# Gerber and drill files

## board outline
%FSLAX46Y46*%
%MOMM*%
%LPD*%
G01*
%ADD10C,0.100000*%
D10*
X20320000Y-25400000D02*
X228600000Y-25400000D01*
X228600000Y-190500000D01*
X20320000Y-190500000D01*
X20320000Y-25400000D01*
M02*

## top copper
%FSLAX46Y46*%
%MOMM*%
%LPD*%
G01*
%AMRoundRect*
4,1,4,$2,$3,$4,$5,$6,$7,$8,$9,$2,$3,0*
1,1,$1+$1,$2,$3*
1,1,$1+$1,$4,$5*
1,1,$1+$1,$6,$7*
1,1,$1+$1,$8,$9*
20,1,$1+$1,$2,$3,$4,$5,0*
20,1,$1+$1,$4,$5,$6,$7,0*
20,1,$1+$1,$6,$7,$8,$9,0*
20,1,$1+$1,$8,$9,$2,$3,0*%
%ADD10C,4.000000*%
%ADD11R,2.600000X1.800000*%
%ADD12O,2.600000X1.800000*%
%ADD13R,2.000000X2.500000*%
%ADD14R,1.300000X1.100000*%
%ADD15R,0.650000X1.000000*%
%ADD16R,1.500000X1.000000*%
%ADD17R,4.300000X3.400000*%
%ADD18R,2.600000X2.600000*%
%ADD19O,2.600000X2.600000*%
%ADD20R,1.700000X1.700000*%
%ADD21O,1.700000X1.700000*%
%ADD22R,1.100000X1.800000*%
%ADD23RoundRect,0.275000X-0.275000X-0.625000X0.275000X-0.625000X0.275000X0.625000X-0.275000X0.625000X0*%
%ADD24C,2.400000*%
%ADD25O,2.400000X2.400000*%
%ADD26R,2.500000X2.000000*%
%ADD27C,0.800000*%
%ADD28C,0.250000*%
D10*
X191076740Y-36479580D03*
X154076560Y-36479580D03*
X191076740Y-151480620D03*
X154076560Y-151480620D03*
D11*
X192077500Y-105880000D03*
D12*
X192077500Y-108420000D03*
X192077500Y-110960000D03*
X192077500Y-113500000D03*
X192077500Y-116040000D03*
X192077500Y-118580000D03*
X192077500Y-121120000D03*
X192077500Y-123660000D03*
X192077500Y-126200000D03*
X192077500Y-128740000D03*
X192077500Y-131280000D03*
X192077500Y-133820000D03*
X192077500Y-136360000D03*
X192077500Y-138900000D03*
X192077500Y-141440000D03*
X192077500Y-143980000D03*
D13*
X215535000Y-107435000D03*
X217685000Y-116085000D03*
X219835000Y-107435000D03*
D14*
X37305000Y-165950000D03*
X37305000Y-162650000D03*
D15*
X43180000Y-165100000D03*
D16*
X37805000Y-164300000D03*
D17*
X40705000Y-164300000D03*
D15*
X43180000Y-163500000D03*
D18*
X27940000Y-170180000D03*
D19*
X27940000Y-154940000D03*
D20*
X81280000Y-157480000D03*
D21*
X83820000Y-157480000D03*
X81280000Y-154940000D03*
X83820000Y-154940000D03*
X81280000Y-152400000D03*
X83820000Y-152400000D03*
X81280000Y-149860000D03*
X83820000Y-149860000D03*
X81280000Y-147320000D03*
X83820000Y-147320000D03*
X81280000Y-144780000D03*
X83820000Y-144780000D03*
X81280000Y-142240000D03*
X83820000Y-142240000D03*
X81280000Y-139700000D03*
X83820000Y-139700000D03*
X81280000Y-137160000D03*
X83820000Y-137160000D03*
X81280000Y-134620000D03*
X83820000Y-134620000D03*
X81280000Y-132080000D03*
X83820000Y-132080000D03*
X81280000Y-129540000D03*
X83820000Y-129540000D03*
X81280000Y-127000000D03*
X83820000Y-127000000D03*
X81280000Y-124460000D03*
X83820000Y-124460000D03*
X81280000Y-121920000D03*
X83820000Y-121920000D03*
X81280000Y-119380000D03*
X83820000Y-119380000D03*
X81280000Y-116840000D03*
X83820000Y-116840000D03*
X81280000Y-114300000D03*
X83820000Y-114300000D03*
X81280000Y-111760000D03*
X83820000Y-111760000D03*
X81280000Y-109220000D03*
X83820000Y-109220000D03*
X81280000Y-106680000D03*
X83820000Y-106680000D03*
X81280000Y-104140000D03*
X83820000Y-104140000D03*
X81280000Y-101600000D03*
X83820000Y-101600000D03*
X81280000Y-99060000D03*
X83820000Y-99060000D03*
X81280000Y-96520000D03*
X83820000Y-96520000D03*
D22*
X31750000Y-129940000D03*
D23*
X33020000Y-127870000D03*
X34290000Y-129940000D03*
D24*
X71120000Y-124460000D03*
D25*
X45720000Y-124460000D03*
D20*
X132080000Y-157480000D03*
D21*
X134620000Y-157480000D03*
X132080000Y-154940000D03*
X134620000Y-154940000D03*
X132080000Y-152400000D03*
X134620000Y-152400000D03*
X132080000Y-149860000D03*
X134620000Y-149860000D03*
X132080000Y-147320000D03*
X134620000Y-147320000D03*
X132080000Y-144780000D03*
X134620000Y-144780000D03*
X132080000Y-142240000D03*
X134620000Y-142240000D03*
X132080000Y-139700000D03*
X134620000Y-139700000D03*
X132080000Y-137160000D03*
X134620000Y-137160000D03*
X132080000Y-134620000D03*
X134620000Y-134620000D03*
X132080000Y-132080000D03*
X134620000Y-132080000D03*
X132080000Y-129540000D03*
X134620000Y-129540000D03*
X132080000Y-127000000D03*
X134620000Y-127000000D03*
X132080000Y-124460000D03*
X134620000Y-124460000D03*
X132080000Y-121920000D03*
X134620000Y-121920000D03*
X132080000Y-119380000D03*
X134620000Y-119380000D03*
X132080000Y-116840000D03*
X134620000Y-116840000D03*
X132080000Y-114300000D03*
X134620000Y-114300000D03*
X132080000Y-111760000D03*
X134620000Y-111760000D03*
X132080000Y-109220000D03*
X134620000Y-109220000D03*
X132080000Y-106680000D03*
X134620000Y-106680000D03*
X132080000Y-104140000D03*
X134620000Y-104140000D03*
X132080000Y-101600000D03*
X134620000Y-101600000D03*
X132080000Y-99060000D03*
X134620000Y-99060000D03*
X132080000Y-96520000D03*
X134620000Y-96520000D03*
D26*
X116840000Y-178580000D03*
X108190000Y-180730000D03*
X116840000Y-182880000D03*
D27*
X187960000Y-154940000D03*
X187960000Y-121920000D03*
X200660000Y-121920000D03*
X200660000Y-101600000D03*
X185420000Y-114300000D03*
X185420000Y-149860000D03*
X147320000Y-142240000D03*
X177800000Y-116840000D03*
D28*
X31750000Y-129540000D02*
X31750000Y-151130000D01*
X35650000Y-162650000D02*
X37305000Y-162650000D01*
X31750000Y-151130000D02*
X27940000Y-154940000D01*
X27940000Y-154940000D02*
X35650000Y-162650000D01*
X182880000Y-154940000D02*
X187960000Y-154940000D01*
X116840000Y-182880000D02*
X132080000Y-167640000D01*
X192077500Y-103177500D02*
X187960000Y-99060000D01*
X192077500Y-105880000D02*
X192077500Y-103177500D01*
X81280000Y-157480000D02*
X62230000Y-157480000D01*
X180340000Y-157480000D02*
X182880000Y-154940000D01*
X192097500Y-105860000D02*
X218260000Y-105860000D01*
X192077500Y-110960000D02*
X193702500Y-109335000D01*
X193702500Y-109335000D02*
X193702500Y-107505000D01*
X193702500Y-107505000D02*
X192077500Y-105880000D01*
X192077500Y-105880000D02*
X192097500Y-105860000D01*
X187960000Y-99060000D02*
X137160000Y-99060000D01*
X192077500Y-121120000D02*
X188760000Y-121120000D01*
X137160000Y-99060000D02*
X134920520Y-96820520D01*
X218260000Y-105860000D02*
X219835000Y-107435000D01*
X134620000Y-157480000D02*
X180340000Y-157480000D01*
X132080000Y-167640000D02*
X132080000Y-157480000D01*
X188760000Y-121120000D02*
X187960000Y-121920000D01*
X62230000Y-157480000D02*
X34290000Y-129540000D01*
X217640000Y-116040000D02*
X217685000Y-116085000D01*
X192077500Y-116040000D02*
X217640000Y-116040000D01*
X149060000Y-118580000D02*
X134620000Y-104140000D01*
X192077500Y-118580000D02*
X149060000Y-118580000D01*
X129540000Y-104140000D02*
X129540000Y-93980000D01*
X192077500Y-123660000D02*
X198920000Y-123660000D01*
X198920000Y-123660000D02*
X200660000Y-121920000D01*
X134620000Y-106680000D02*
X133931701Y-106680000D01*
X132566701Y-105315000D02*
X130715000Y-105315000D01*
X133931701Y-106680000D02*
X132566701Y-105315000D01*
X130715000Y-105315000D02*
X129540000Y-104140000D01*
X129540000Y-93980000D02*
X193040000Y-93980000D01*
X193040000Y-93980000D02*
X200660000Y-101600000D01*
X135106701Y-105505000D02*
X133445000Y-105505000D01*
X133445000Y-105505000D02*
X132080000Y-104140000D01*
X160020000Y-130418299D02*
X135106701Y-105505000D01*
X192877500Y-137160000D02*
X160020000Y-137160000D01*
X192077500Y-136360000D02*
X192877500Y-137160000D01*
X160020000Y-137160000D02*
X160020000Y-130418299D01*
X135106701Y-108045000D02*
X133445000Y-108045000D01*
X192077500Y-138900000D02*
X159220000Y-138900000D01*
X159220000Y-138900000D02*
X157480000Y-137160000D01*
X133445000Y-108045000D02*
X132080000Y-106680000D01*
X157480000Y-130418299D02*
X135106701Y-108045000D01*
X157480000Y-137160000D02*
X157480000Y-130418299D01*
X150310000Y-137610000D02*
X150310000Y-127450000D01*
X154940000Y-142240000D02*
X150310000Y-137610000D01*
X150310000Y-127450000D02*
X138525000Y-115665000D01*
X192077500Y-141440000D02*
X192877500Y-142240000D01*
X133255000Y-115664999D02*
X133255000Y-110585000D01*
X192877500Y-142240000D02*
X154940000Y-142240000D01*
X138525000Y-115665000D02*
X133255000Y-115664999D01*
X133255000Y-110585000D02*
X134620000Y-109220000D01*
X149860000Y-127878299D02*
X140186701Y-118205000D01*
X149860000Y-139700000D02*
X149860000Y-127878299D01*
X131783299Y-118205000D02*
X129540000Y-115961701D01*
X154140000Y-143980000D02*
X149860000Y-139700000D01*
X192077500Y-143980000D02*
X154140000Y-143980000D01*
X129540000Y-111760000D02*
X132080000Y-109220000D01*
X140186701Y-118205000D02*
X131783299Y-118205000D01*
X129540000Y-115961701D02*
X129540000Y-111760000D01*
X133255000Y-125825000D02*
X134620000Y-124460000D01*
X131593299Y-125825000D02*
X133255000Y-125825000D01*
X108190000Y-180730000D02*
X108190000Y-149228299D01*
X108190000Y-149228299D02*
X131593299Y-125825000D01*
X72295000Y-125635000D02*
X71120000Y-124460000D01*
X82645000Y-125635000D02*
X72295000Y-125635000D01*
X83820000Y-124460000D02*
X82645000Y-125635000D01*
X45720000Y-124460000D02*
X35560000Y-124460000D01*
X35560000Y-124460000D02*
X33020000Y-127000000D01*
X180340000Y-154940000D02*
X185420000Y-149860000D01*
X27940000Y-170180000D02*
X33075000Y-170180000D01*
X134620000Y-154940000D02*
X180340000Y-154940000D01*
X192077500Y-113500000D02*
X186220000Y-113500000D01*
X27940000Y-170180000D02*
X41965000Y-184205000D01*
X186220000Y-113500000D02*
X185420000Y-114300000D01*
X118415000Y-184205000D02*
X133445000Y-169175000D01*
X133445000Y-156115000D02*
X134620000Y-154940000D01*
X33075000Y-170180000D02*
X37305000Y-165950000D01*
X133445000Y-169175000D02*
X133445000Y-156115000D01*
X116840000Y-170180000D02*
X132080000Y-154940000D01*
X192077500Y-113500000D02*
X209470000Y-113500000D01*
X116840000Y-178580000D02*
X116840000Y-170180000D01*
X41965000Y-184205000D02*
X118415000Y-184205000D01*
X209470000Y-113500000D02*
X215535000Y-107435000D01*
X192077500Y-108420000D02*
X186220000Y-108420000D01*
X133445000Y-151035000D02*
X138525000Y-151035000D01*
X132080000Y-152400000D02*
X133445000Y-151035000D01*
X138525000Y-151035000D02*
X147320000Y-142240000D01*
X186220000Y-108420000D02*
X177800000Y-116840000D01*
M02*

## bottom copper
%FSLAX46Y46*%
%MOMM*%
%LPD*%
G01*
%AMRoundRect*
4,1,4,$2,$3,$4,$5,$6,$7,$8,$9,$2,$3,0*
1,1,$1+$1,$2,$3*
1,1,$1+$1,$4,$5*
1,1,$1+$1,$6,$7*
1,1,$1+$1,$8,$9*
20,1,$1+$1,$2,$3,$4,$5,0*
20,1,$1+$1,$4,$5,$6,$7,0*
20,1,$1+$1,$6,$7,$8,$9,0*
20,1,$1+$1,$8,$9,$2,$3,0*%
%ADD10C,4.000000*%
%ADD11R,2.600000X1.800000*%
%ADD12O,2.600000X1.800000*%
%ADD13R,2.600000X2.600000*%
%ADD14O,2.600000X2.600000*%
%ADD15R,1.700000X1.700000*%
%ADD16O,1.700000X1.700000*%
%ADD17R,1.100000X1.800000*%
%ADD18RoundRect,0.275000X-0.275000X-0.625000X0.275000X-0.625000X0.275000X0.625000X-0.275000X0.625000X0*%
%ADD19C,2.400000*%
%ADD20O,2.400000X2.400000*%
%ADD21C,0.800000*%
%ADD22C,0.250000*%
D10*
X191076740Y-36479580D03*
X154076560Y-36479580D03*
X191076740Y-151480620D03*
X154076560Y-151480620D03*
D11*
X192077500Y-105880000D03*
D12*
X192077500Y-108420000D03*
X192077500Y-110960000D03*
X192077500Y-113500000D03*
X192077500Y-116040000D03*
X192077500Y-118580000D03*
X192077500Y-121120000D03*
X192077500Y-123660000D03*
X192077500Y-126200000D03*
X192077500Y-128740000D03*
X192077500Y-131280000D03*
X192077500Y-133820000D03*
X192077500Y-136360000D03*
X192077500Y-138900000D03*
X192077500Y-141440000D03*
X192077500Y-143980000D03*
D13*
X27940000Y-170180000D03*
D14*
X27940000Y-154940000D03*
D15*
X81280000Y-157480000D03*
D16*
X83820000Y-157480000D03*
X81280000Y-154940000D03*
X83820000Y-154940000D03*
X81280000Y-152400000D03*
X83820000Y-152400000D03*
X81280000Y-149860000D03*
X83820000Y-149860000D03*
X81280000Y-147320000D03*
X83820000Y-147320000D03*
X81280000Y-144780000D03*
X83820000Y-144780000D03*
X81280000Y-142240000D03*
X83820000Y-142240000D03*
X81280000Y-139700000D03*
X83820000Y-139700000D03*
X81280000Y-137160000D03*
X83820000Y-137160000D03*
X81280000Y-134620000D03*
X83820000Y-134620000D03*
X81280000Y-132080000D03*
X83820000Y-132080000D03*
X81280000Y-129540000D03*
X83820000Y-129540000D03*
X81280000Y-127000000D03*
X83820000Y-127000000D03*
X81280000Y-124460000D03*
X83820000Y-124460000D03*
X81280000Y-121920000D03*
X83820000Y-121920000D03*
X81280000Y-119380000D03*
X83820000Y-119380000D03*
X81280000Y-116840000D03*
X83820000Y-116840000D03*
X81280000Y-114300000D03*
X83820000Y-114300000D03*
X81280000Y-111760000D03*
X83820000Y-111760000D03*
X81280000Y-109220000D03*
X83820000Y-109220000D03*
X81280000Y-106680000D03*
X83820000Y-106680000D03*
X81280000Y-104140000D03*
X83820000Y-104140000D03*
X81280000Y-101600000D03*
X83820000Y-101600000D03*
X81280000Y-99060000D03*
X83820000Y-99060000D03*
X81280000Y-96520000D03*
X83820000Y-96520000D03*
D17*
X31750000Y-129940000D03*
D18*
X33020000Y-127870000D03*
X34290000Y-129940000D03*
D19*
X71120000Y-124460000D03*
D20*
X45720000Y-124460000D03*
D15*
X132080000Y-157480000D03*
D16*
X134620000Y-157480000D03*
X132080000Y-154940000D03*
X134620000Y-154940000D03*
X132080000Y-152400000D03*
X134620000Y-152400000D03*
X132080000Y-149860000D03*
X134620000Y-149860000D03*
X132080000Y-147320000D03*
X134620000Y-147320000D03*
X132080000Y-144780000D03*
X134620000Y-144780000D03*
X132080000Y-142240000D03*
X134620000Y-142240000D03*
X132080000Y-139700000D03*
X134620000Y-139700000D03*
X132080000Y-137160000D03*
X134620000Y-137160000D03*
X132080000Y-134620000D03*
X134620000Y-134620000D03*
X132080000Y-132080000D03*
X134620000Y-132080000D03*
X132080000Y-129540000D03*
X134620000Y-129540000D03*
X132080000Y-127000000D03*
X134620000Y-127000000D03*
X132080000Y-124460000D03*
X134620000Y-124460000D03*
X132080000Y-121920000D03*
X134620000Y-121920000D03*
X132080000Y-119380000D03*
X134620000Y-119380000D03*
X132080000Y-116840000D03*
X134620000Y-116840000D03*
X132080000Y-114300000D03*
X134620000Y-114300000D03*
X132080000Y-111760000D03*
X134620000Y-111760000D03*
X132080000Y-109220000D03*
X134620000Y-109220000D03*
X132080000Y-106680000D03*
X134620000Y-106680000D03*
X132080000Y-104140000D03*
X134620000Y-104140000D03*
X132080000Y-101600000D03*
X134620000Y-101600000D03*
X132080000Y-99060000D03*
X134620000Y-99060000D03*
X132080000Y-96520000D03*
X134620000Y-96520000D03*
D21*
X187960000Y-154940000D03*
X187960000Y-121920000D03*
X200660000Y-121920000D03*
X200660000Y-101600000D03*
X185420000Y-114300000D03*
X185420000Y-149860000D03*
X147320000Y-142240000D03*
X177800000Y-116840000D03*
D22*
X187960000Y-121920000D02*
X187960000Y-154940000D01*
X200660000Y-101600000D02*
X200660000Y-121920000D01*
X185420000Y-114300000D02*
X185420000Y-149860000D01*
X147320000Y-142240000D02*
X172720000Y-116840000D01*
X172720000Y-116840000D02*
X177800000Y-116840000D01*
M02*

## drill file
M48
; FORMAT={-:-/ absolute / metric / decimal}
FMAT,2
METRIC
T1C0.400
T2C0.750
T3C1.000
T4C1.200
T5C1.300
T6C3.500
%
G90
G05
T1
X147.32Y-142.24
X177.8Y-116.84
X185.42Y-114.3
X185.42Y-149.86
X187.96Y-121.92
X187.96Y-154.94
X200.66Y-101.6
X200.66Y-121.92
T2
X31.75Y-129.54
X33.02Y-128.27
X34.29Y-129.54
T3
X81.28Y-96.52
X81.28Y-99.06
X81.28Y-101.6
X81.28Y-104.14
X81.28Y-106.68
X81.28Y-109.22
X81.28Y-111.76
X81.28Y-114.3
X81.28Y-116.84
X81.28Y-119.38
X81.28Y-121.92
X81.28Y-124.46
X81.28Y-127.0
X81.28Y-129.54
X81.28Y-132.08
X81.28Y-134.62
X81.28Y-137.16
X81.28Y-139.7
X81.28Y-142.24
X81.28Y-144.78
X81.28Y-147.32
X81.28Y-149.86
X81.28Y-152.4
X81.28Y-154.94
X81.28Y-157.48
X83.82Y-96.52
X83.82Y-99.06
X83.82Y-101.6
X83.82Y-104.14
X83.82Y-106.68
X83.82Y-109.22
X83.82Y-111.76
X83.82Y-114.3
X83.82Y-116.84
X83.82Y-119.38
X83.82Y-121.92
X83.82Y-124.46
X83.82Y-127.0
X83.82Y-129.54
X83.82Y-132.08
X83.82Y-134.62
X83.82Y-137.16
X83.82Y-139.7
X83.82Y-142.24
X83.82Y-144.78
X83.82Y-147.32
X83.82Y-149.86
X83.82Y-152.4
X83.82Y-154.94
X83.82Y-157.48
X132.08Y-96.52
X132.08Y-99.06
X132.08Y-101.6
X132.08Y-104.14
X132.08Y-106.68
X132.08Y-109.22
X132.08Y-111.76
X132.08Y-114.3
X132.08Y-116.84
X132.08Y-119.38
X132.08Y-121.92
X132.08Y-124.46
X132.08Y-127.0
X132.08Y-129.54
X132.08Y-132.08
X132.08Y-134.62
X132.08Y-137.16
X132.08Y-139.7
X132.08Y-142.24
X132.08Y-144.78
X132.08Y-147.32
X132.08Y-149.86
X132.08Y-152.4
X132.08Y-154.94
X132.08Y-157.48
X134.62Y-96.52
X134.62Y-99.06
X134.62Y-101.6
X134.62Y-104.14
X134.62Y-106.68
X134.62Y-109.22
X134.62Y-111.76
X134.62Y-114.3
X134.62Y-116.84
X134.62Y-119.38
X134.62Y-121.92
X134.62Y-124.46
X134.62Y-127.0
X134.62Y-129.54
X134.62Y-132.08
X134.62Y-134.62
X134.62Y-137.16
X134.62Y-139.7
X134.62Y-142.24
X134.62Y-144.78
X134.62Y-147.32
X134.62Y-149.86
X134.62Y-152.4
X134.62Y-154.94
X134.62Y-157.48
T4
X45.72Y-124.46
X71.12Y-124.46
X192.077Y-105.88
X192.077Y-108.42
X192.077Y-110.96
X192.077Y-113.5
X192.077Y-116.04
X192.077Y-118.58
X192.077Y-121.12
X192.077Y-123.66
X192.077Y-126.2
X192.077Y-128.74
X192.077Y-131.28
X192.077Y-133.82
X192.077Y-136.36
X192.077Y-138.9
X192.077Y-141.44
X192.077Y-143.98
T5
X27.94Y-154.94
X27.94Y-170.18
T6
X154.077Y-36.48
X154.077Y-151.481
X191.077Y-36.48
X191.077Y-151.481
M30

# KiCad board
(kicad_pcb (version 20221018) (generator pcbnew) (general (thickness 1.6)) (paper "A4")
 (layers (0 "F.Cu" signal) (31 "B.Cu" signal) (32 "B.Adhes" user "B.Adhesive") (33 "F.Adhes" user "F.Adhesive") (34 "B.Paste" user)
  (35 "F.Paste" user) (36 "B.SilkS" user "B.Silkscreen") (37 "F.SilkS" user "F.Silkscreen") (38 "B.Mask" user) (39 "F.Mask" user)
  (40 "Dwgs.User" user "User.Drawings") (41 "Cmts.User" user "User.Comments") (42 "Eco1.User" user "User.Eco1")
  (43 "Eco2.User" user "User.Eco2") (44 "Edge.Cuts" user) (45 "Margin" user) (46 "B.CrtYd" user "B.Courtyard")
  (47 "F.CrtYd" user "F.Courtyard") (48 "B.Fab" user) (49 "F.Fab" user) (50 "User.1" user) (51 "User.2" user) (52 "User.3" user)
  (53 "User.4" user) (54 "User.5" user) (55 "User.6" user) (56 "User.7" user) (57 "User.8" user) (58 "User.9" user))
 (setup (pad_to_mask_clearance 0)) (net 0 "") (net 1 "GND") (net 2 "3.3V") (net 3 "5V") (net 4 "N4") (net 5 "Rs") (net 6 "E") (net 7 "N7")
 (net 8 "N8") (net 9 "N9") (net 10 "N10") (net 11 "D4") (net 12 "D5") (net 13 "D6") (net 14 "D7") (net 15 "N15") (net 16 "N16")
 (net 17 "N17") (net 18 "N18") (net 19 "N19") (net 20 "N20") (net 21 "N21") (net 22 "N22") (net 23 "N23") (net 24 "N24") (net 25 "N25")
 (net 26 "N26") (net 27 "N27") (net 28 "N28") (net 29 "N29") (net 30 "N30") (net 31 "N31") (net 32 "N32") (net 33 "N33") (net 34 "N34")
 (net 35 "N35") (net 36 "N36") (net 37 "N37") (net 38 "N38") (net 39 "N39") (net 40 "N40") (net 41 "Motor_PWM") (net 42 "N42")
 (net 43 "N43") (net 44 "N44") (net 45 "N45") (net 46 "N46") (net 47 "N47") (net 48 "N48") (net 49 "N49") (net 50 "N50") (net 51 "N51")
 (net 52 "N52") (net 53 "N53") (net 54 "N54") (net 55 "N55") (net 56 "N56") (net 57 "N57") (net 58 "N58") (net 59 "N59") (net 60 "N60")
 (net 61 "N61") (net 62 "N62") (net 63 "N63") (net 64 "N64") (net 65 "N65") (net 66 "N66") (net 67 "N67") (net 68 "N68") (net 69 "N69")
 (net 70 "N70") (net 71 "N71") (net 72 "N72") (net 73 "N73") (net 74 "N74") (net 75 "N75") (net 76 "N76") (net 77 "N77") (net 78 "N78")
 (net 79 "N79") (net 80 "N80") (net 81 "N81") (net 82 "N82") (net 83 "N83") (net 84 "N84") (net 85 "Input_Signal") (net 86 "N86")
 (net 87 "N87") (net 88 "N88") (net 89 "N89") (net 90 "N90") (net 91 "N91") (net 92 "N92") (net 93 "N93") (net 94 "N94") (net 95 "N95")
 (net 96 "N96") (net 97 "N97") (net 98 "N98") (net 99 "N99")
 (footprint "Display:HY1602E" (layer "F.Cu") (at 192.0775 105.88 -90)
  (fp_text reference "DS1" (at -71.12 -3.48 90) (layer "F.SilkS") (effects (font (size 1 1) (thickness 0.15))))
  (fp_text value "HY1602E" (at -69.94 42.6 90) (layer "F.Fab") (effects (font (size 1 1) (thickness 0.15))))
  (pad "" thru_hole circle (at -69.40042 1.00076 90) (size 4 4) (drill 3.5) (layers "*.Cu" "*.Mask"))
  (pad "" thru_hole circle (at -69.40042 38.00094 90) (size 4 4) (drill 3.5) (layers "*.Cu" "*.Mask"))
  (pad "" thru_hole circle (at 45.60062 1.00076 90) (size 4 4) (drill 3.5) (layers "*.Cu" "*.Mask"))
  (pad "" thru_hole circle (at 45.60062 38.00094 90) (size 4 4) (drill 3.5) (layers "*.Cu" "*.Mask"))
  (pad "1" thru_hole rect (at 0 0 90) (size 1.8 2.6) (drill 1.2) (layers "*.Cu" "*.Mask") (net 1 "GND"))
  (pad "2" thru_hole oval (at 2.54 0 90) (size 1.8 2.6) (drill 1.2) (layers "*.Cu" "*.Mask") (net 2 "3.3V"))
  (pad "3" thru_hole oval (at 5.08 0 90) (size 1.8 2.6) (drill 1.2) (layers "*.Cu" "*.Mask") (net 1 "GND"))
  (pad "4" thru_hole oval (at 7.62 0 90) (size 1.8 2.6) (drill 1.2) (layers "*.Cu" "*.Mask") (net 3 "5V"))
  (pad "5" thru_hole oval (at 10.16 0 90) (size 1.8 2.6) (drill 1.2) (layers "*.Cu" "*.Mask") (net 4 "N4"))
  (pad "6" thru_hole oval (at 12.7 0 90) (size 1.8 2.6) (drill 1.2) (layers "*.Cu" "*.Mask") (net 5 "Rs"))
  (pad "7" thru_hole oval (at 15.24 0 90) (size 1.8 2.6) (drill 1.2) (layers "*.Cu" "*.Mask") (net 1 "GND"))
  (pad "8" thru_hole oval (at 17.78 0 90) (size 1.8 2.6) (drill 1.2) (layers "*.Cu" "*.Mask") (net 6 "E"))
  (pad "9" thru_hole oval (at 20.32 0 90) (size 1.8 2.6) (drill 1.2) (layers "*.Cu" "*.Mask") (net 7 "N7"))
  (pad "10" thru_hole oval (at 22.86 0 90) (size 1.8 2.6) (drill 1.2) (layers "*.Cu" "*.Mask") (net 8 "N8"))
  (pad "11" thru_hole oval (at 25.4 0 90) (size 1.8 2.6) (drill 1.2) (layers "*.Cu" "*.Mask") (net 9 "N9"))
  (pad "12" thru_hole oval (at 27.94 0 90) (size 1.8 2.6) (drill 1.2) (layers "*.Cu" "*.Mask") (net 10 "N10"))
  (pad "13" thru_hole oval (at 30.48 0 90) (size 1.8 2.6) (drill 1.2) (layers "*.Cu" "*.Mask") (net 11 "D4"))
  (pad "14" thru_hole oval (at 33.02 0 90) (size 1.8 2.6) (drill 1.2) (layers "*.Cu" "*.Mask") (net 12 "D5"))
  (pad "15" thru_hole oval (at 35.56 0 90) (size 1.8 2.6) (drill 1.2) (layers "*.Cu" "*.Mask") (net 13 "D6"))
  (pad "16" thru_hole oval (at 38.1 0 90) (size 1.8 2.6) (drill 1.2) (layers "*.Cu" "*.Mask") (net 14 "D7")))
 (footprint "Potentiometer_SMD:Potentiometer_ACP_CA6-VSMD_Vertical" (layer "F.Cu") (at 217.685 111.76 -90)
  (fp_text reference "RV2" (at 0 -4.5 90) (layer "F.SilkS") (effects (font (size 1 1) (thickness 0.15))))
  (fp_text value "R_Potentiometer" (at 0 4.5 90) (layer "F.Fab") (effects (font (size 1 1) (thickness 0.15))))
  (pad "1" smd rect (at -4.325 2.15 270) (size 2.5 2) (layers "F.Cu" "F.Paste" "F.Mask") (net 3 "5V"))
  (pad "2" smd rect (at 4.325 0 270) (size 2.5 2) (layers "F.Cu" "F.Paste" "F.Mask") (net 4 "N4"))
  (pad "3" smd rect (at -4.325 -2.15 270) (size 2.5 2) (layers "F.Cu" "F.Paste" "F.Mask") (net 1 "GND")))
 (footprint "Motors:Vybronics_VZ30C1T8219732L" (layer "F.Cu") (at 41.655 164.3 90)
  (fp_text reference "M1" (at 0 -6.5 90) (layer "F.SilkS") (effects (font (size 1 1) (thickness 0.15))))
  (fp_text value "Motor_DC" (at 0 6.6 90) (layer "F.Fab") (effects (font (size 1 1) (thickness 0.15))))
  (pad "" smd rect (at -0.85 -2.315) (size 1.07 1.4) (layers "F.Paste"))
  (pad "" smd rect (at -0.85 -0.905) (size 1.07 1.4) (layers "F.Paste"))
  (pad "" smd rect (at -0.85 0.505) (size 1.07 1.4) (layers "F.Paste"))
  (pad "" smd rect (at 0.85 -2.315) (size 1.07 1.4) (layers "F.Paste"))
  (pad "" smd rect (at 0.85 -0.905) (size 1.07 1.4) (layers "F.Paste"))
  (pad "" smd rect (at 0.85 0.505) (size 1.07 1.4) (layers "F.Paste"))
  (pad "1" smd rect (at -1.65 -4.35) (size 1.3 1.1) (layers "F.Cu" "F.Paste" "F.Mask") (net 3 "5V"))
  (pad "2" smd rect (at 1.65 -4.35) (size 1.3 1.1) (layers "F.Cu" "F.Paste" "F.Mask") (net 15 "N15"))
  (pad "SH" smd rect (at -0.8 1.525 90) (size 1 0.65) (layers "F.Cu" "F.Paste" "F.Mask"))
  (pad "SH" smd rect (at 0 -3.85) (size 1.5 1) (layers "F.Cu" "F.Paste" "F.Mask"))
  (pad "SH" smd rect (at 0 -0.95) (size 4.3 3.4) (layers "F.Cu" "F.Mask"))
  (pad "SH" smd rect (at 0.8 1.525 90) (size 1 0.65) (layers "F.Cu" "F.Paste" "F.Mask")))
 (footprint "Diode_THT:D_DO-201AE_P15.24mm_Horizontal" (layer "F.Cu") (at 27.94 170.18 90)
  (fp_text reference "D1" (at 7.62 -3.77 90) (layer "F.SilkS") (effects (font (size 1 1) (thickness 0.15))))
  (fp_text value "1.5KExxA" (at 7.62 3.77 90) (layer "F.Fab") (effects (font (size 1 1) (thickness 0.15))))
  (pad "1" thru_hole rect (at 0 0 90) (size 2.6 2.6) (drill 1.3) (layers "*.Cu" "*.Mask") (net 3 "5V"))
  (pad "2" thru_hole oval (at 15.24 0 90) (size 2.6 2.6) (drill 1.3) (layers "*.Cu" "*.Mask") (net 15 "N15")))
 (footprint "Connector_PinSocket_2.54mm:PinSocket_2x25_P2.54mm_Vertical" (layer "F.Cu") (at 81.28 157.48 180)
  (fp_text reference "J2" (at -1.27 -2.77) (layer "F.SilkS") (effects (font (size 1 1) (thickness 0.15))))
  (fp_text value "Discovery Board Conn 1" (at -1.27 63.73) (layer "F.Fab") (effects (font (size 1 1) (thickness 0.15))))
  (pad "1" thru_hole rect (at 0 0 180) (size 1.7 1.7) (drill 1) (layers "*.Cu" "*.Mask") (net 1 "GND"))
  (pad "2" thru_hole oval (at -2.54 0 180) (size 1.7 1.7) (drill 1) (layers "*.Cu" "*.Mask") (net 1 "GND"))
  (pad "3" thru_hole oval (at 0 2.54 180) (size 1.7 1.7) (drill 1) (layers "*.Cu" "*.Mask") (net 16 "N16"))
  (pad "4" thru_hole oval (at -2.54 2.54 180) (size 1.7 1.7) (drill 1) (layers "*.Cu" "*.Mask") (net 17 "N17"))
  (pad "5" thru_hole oval (at 0 5.08 180) (size 1.7 1.7) (drill 1) (layers "*.Cu" "*.Mask") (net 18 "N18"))
  (pad "6" thru_hole oval (at -2.54 5.08 180) (size 1.7 1.7) (drill 1) (layers "*.Cu" "*.Mask") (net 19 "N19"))
  (pad "7" thru_hole oval (at 0 7.62 180) (size 1.7 1.7) (drill 1) (layers "*.Cu" "*.Mask") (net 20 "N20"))
  (pad "8" thru_hole oval (at -2.54 7.62 180) (size 1.7 1.7) (drill 1) (layers "*.Cu" "*.Mask") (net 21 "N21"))
  (pad "9" thru_hole oval (at 0 10.16 180) (size 1.7 1.7) (drill 1) (layers "*.Cu" "*.Mask") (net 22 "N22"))
  (pad "10" thru_hole oval (at -2.54 10.16 180) (size 1.7 1.7) (drill 1) (layers "*.Cu" "*.Mask") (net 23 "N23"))
  (pad "11" thru_hole oval (at 0 12.7 180) (size 1.7 1.7) (drill 1) (layers "*.Cu" "*.Mask") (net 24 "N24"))
  (pad "12" thru_hole oval (at -2.54 12.7 180) (size 1.7 1.7) (drill 1) (layers "*.Cu" "*.Mask") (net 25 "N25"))
  (pad "13" thru_hole oval (at 0 15.24 180) (size 1.7 1.7) (drill 1) (layers "*.Cu" "*.Mask") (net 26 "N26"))
  (pad "14" thru_hole oval (at -2.54 15.24 180) (size 1.7 1.7) (drill 1) (layers "*.Cu" "*.Mask") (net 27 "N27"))
  (pad "15" thru_hole oval (at 0 17.78 180) (size 1.7 1.7) (drill 1) (layers "*.Cu" "*.Mask") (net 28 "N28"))
  (pad "16" thru_hole oval (at -2.54 17.78 180) (size 1.7 1.7) (drill 1) (layers "*.Cu" "*.Mask") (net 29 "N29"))
  (pad "17" thru_hole oval (at 0 20.32 180) (size 1.7 1.7) (drill 1) (layers "*.Cu" "*.Mask") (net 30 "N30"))
  (pad "18" thru_hole oval (at -2.54 20.32 180) (size 1.7 1.7) (drill 1) (layers "*.Cu" "*.Mask") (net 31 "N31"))
  (pad "19" thru_hole oval (at 0 22.86 180) (size 1.7 1.7) (drill 1) (layers "*.Cu" "*.Mask") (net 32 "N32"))
  (pad "20" thru_hole oval (at -2.54 22.86 180) (size 1.7 1.7) (drill 1) (layers "*.Cu" "*.Mask") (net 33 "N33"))
  (pad "21" thru_hole oval (at 0 25.4 180) (size 1.7 1.7) (drill 1) (layers "*.Cu" "*.Mask") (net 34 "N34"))
  (pad "22" thru_hole oval (at -2.54 25.4 180) (size 1.7 1.7) (drill 1) (layers "*.Cu" "*.Mask") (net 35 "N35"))
  (pad "23" thru_hole oval (at 0 27.94 180) (size 1.7 1.7) (drill 1) (layers "*.Cu" "*.Mask") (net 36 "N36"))
  (pad "24" thru_hole oval (at -2.54 27.94 180) (size 1.7 1.7) (drill 1) (layers "*.Cu" "*.Mask") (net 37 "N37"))
  (pad "25" thru_hole oval (at 0 30.48 180) (size 1.7 1.7) (drill 1) (layers "*.Cu" "*.Mask") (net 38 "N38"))
  (pad "26" thru_hole oval (at -2.54 30.48 180) (size 1.7 1.7) (drill 1) (layers "*.Cu" "*.Mask") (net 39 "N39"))
  (pad "27" thru_hole oval (at 0 33.02 180) (size 1.7 1.7) (drill 1) (layers "*.Cu" "*.Mask") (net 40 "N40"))
  (pad "28" thru_hole oval (at -2.54 33.02 180) (size 1.7 1.7) (drill 1) (layers "*.Cu" "*.Mask") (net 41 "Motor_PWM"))
  (pad "29" thru_hole oval (at 0 35.56 180) (size 1.7 1.7) (drill 1) (layers "*.Cu" "*.Mask") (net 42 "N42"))
  (pad "30" thru_hole oval (at -2.54 35.56 180) (size 1.7 1.7) (drill 1) (layers "*.Cu" "*.Mask") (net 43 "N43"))
  (pad "31" thru_hole oval (at 0 38.1 180) (size 1.7 1.7) (drill 1) (layers "*.Cu" "*.Mask") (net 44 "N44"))
  (pad "32" thru_hole oval (at -2.54 38.1 180) (size 1.7 1.7) (drill 1) (layers "*.Cu" "*.Mask") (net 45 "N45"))
  (pad "33" thru_hole oval (at 0 40.64 180) (size 1.7 1.7) (drill 1) (layers "*.Cu" "*.Mask") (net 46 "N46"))
  (pad "34" thru_hole oval (at -2.54 40.64 180) (size 1.7 1.7) (drill 1) (layers "*.Cu" "*.Mask") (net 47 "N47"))
  (pad "35" thru_hole oval (at 0 43.18 180) (size 1.7 1.7) (drill 1) (layers "*.Cu" "*.Mask") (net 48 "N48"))
  (pad "36" thru_hole oval (at -2.54 43.18 180) (size 1.7 1.7) (drill 1) (layers "*.Cu" "*.Mask") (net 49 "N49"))
  (pad "37" thru_hole oval (at 0 45.72 180) (size 1.7 1.7) (drill 1) (layers "*.Cu" "*.Mask") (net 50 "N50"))
  (pad "38" thru_hole oval (at -2.54 45.72 180) (size 1.7 1.7) (drill 1) (layers "*.Cu" "*.Mask") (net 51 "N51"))
  (pad "39" thru_hole oval (at 0 48.26 180) (size 1.7 1.7) (drill 1) (layers "*.Cu" "*.Mask") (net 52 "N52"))
  (pad "40" thru_hole oval (at -2.54 48.26 180) (size 1.7 1.7) (drill 1) (layers "*.Cu" "*.Mask") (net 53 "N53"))
  (pad "41" thru_hole oval (at 0 50.8 180) (size 1.7 1.7) (drill 1) (layers "*.Cu" "*.Mask") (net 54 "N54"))
  (pad "42" thru_hole oval (at -2.54 50.8 180) (size 1.7 1.7) (drill 1) (layers "*.Cu" "*.Mask") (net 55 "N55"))
  (pad "43" thru_hole oval (at 0 53.34 180) (size 1.7 1.7) (drill 1) (layers "*.Cu" "*.Mask") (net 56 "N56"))
  (pad "44" thru_hole oval (at -2.54 53.34 180) (size 1.7 1.7) (drill 1) (layers "*.Cu" "*.Mask") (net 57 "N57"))
  (pad "45" thru_hole oval (at 0 55.88 180) (size 1.7 1.7) (drill 1) (layers "*.Cu" "*.Mask") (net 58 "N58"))
  (pad "46" thru_hole oval (at -2.54 55.88 180) (size 1.7 1.7) (drill 1) (layers "*.Cu" "*.Mask") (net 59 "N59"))
  (pad "47" thru_hole oval (at 0 58.42 180) (size 1.7 1.7) (drill 1) (layers "*.Cu" "*.Mask") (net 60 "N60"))
  (pad "48" thru_hole oval (at -2.54 58.42 180) (size 1.7 1.7) (drill 1) (layers "*.Cu" "*.Mask") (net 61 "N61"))
  (pad "49" thru_hole oval (at 0 60.96 180) (size 1.7 1.7) (drill 1) (layers "*.Cu" "*.Mask") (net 1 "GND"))
  (pad "50" thru_hole oval (at -2.54 60.96 180) (size 1.7 1.7) (drill 1) (layers "*.Cu" "*.Mask") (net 1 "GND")))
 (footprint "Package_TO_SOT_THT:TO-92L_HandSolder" (layer "F.Cu") (at 31.75 129.54)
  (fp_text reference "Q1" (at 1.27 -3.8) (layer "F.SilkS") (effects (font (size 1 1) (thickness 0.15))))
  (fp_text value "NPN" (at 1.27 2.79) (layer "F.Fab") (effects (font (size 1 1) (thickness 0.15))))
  (pad "1" thru_hole rect (at 0 0) (size 1.1 1.8) (drill 0.75 (offset 0 0.4)) (layers "*.Cu" "*.Mask") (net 15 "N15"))
  (pad "2" thru_hole roundrect (at 1.27 -1.27) (size 1.1 1.8) (drill 0.75 (offset 0 -0.4)) (layers "*.Cu" "*.Mask") (roundrect_rratio 0.25)
   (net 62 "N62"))
  (pad "3" thru_hole roundrect (at 2.54 0) (size 1.1 1.8) (drill 0.75 (offset 0 0.4)) (layers "*.Cu" "*.Mask") (roundrect_rratio 0.25)
   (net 1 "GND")))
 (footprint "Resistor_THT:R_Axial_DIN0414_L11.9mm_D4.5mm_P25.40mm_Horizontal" (layer "F.Cu") (at 71.12 124.46 180)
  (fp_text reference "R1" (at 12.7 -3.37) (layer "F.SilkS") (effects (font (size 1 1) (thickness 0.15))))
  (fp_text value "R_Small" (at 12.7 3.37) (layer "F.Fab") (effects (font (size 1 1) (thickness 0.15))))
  (pad "1" thru_hole circle (at 0 0 180) (size 2.4 2.4) (drill 1.2) (layers "*.Cu" "*.Mask") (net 41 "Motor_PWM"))
  (pad "2" thru_hole oval (at 25.4 0 180) (size 2.4 2.4) (drill 1.2) (layers "*.Cu" "*.Mask") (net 62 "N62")))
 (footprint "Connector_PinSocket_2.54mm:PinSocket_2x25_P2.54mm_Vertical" (layer "F.Cu") (at 132.08 157.48 180)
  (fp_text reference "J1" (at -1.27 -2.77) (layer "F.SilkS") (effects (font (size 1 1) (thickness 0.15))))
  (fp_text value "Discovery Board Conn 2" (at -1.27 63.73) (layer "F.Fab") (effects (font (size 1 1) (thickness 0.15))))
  (pad "1" thru_hole rect (at 0 0 180) (size 1.7 1.7) (drill 1) (layers "*.Cu" "*.Mask") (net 1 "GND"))
  (pad "2" thru_hole oval (at -2.54 0 180) (size 1.7 1.7) (drill 1) (layers "*.Cu" "*.Mask") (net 1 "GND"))
  (pad "3" thru_hole oval (at 0 2.54 180) (size 1.7 1.7) (drill 1) (layers "*.Cu" "*.Mask") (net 3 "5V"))
  (pad "4" thru_hole oval (at -2.54 2.54 180) (size 1.7 1.7) (drill 1) (layers "*.Cu" "*.Mask") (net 3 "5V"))
  (pad "5" thru_hole oval (at 0 5.08 180) (size 1.7 1.7) (drill 1) (layers "*.Cu" "*.Mask") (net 2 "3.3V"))
  (pad "6" thru_hole oval (at -2.54 5.08 180) (size 1.7 1.7) (drill 1) (layers "*.Cu" "*.Mask") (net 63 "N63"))
  (pad "7" thru_hole oval (at 0 7.62 180) (size 1.7 1.7) (drill 1) (layers "*.Cu" "*.Mask") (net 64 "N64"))
  (pad "8" thru_hole oval (at -2.54 7.62 180) (size 1.7 1.7) (drill 1) (layers "*.Cu" "*.Mask") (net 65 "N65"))
  (pad "9" thru_hole oval (at 0 10.16 180) (size 1.7 1.7) (drill 1) (layers "*.Cu" "*.Mask") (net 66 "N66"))
  (pad "10" thru_hole oval (at -2.54 10.16 180) (size 1.7 1.7) (drill 1) (layers "*.Cu" "*.Mask") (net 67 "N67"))
  (pad "11" thru_hole oval (at 0 12.7 180) (size 1.7 1.7) (drill 1) (layers "*.Cu" "*.Mask") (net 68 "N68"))
  (pad "12" thru_hole oval (at -2.54 12.7 180) (size 1.7 1.7) (drill 1) (layers "*.Cu" "*.Mask") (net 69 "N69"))
  (pad "13" thru_hole oval (at 0 15.24 180) (size 1.7 1.7) (drill 1) (layers "*.Cu" "*.Mask") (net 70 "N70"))
  (pad "14" thru_hole oval (at -2.54 15.24 180) (size 1.7 1.7) (drill 1) (layers "*.Cu" "*.Mask") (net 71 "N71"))
  (pad "15" thru_hole oval (at 0 17.78 180) (size 1.7 1.7) (drill 1) (layers "*.Cu" "*.Mask") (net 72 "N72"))
  (pad "16" thru_hole oval (at -2.54 17.78 180) (size 1.7 1.7) (drill 1) (layers "*.Cu" "*.Mask") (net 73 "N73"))
  (pad "17" thru_hole oval (at 0 20.32 180) (size 1.7 1.7) (drill 1) (layers "*.Cu" "*.Mask") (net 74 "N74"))
  (pad "18" thru_hole oval (at -2.54 20.32 180) (size 1.7 1.7) (drill 1) (layers "*.Cu" "*.Mask") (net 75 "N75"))
  (pad "19" thru_hole oval (at 0 22.86 180) (size 1.7 1.7) (drill 1) (layers "*.Cu" "*.Mask") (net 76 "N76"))
  (pad "20" thru_hole oval (at -2.54 22.86 180) (size 1.7 1.7) (drill 1) (layers "*.Cu" "*.Mask") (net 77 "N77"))
  (pad "21" thru_hole oval (at 0 25.4 180) (size 1.7 1.7) (drill 1) (layers "*.Cu" "*.Mask") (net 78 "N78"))
  (pad "22" thru_hole oval (at -2.54 25.4 180) (size 1.7 1.7) (drill 1) (layers "*.Cu" "*.Mask") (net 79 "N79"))
  (pad "23" thru_hole oval (at 0 27.94 180) (size 1.7 1.7) (drill 1) (layers "*.Cu" "*.Mask") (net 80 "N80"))
  (pad "24" thru_hole oval (at -2.54 27.94 180) (size 1.7 1.7) (drill 1) (layers "*.Cu" "*.Mask") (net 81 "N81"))
  (pad "25" thru_hole oval (at 0 30.48 180) (size 1.7 1.7) (drill 1) (layers "*.Cu" "*.Mask") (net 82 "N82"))
  (pad "26" thru_hole oval (at -2.54 30.48 180) (size 1.7 1.7) (drill 1) (layers "*.Cu" "*.Mask") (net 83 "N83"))
  (pad "27" thru_hole oval (at 0 33.02 180) (size 1.7 1.7) (drill 1) (layers "*.Cu" "*.Mask") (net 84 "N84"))
  (pad "28" thru_hole oval (at -2.54 33.02 180) (size 1.7 1.7) (drill 1) (layers "*.Cu" "*.Mask") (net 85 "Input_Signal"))
  (pad "29" thru_hole oval (at 0 35.56 180) (size 1.7 1.7) (drill 1) (layers "*.Cu" "*.Mask") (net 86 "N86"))
  (pad "30" thru_hole oval (at -2.54 35.56 180) (size 1.7 1.7) (drill 1) (layers "*.Cu" "*.Mask") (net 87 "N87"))
  (pad "31" thru_hole oval (at 0 38.1 180) (size 1.7 1.7) (drill 1) (layers "*.Cu" "*.Mask") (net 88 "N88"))
  (pad "32" thru_hole oval (at -2.54 38.1 180) (size 1.7 1.7) (drill 1) (layers "*.Cu" "*.Mask") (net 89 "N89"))
  (pad "33" thru_hole oval (at 0 40.64 180) (size 1.7 1.7) (drill 1) (layers "*.Cu" "*.Mask") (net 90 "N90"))
  (pad "34" thru_hole oval (at -2.54 40.64 180) (size 1.7 1.7) (drill 1) (layers "*.Cu" "*.Mask") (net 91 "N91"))
  (pad "35" thru_hole oval (at 0 43.18 180) (size 1.7 1.7) (drill 1) (layers "*.Cu" "*.Mask") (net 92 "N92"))
  (pad "36" thru_hole oval (at -2.54 43.18 180) (size 1.7 1.7) (drill 1) (layers "*.Cu" "*.Mask") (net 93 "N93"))
  (pad "37" thru_hole oval (at 0 45.72 180) (size 1.7 1.7) (drill 1) (layers "*.Cu" "*.Mask") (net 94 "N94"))
  (pad "38" thru_hole oval (at -2.54 45.72 180) (size 1.7 1.7) (drill 1) (layers "*.Cu" "*.Mask") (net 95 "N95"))
  (pad "39" thru_hole oval (at 0 48.26 180) (size 1.7 1.7) (drill 1) (layers "*.Cu" "*.Mask") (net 14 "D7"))
  (pad "40" thru_hole oval (at -2.54 48.26 180) (size 1.7 1.7) (drill 1) (layers "*.Cu" "*.Mask") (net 13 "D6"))
  (pad "41" thru_hole oval (at 0 50.8 180) (size 1.7 1.7) (drill 1) (layers "*.Cu" "*.Mask") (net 12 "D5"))
  (pad "42" thru_hole oval (at -2.54 50.8 180) (size 1.7 1.7) (drill 1) (layers "*.Cu" "*.Mask") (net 6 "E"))
  (pad "43" thru_hole oval (at 0 53.34 180) (size 1.7 1.7) (drill 1) (layers "*.Cu" "*.Mask") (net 11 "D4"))
  (pad "44" thru_hole oval (at -2.54 53.34 180) (size 1.7 1.7) (drill 1) (layers "*.Cu" "*.Mask") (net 5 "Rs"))
  (pad "45" thru_hole oval (at 0 55.88 180) (size 1.7 1.7) (drill 1) (layers "*.Cu" "*.Mask") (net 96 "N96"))
  (pad "46" thru_hole oval (at -2.54 55.88 180) (size 1.7 1.7) (drill 1) (layers "*.Cu" "*.Mask") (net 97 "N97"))
  (pad "47" thru_hole oval (at 0 58.42 180) (size 1.7 1.7) (drill 1) (layers "*.Cu" "*.Mask") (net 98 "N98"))
  (pad "48" thru_hole oval (at -2.54 58.42 180) (size 1.7 1.7) (drill 1) (layers "*.Cu" "*.Mask") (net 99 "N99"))
  (pad "49" thru_hole oval (at 0 60.96 180) (size 1.7 1.7) (drill 1) (layers "*.Cu" "*.Mask") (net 1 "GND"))
  (pad "50" thru_hole oval (at -2.54 60.96 180) (size 1.7 1.7) (drill 1) (layers "*.Cu" "*.Mask") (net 1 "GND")))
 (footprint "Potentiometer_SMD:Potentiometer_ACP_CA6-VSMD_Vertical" (layer "F.Cu") (at 112.515 180.73 180)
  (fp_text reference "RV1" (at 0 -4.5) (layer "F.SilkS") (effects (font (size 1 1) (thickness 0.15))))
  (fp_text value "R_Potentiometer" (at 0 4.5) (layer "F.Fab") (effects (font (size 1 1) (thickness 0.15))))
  (pad "1" smd rect (at -4.325 2.15 180) (size 2.5 2) (layers "F.Cu" "F.Paste" "F.Mask") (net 3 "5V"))
  (pad "2" smd rect (at 4.325 0 180) (size 2.5 2) (layers "F.Cu" "F.Paste" "F.Mask") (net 85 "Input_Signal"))
  (pad "3" smd rect (at -4.325 -2.15 180) (size 2.5 2) (layers "F.Cu" "F.Paste" "F.Mask") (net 1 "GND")))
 (gr_rect (start 20.32 25.4) (end 228.6 190.5) (stroke (width 0.1) (type default)) (fill none) (layer "Edge.Cuts"))
 (segment (start 31.75 129.54) (end 31.75 151.13) (width 0.25) (layer "F.Cu") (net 15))
 (segment (start 35.65 162.65) (end 37.305 162.65) (width 0.25) (layer "F.Cu") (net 15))
 (segment (start 31.75 151.13) (end 27.94 154.94) (width 0.25) (layer "F.Cu") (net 15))
 (segment (start 27.94 154.94) (end 35.65 162.65) (width 0.25) (layer "F.Cu") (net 15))
 (segment (start 182.88 154.94) (end 187.96 154.94) (width 0.25) (layer "F.Cu") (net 1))
 (segment (start 116.84 182.88) (end 132.08 167.64) (width 0.25) (layer "F.Cu") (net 1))
 (segment (start 192.0775 103.1775) (end 187.96 99.06) (width 0.25) (layer "F.Cu") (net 1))
 (segment (start 192.0775 105.88) (end 192.0775 103.1775) (width 0.25) (layer "F.Cu") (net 1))
 (segment (start 81.28 157.48) (end 62.23 157.48) (width 0.25) (layer "F.Cu") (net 1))
 (segment (start 180.34 157.48) (end 182.88 154.94) (width 0.25) (layer "F.Cu") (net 1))
 (segment (start 192.0975 105.86) (end 218.26 105.86) (width 0.25) (layer "F.Cu") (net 1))
 (segment (start 192.0775 110.96) (end 193.7025 109.335) (width 0.25) (layer "F.Cu") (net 1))
 (segment (start 193.7025 109.335) (end 193.7025 107.505) (width 0.25) (layer "F.Cu") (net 1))
 (segment (start 193.7025 107.505) (end 192.0775 105.88) (width 0.25) (layer "F.Cu") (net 1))
 (segment (start 192.0775 105.88) (end 192.0975 105.86) (width 0.25) (layer "F.Cu") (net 1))
 (segment (start 187.96 99.06) (end 137.16 99.06) (width 0.25) (layer "F.Cu") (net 1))
 (segment (start 192.0775 121.12) (end 188.76 121.12) (width 0.25) (layer "F.Cu") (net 1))
 (segment (start 137.16 99.06) (end 134.92052 96.82052) (width 0.25) (layer "F.Cu") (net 1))
 (segment (start 218.26 105.86) (end 219.835 107.435) (width 0.25) (layer "F.Cu") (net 1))
 (segment (start 134.62 157.48) (end 180.34 157.48) (width 0.25) (layer "F.Cu") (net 1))
 (segment (start 132.08 167.64) (end 132.08 157.48) (width 0.25) (layer "F.Cu") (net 1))
 (segment (start 188.76 121.12) (end 187.96 121.92) (width 0.25) (layer "F.Cu") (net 1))
 (segment (start 62.23 157.48) (end 34.29 129.54) (width 0.25) (layer "F.Cu") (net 1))
 (via (at 187.96 154.94) (size 0.8) (drill 0.4) (layers "F.Cu" "B.Cu") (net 1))
 (via (at 187.96 121.92) (size 0.8) (drill 0.4) (layers "F.Cu" "B.Cu") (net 1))
 (segment (start 187.96 121.92) (end 187.96 154.94) (width 0.25) (layer "B.Cu") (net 1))
 (segment (start 217.64 116.04) (end 217.685 116.085) (width 0.25) (layer "F.Cu") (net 4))
 (segment (start 192.0775 116.04) (end 217.64 116.04) (width 0.25) (layer "F.Cu") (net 4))
 (segment (start 149.06 118.58) (end 134.62 104.14) (width 0.25) (layer "F.Cu") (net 5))
 (segment (start 192.0775 118.58) (end 149.06 118.58) (width 0.25) (layer "F.Cu") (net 5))
 (segment (start 129.54 104.14) (end 129.54 93.98) (width 0.25) (layer "F.Cu") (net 6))
 (segment (start 192.0775 123.66) (end 198.92 123.66) (width 0.25) (layer "F.Cu") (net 6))
 (segment (start 198.92 123.66) (end 200.66 121.92) (width 0.25) (layer "F.Cu") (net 6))
 (segment (start 134.62 106.68) (end 133.931701 106.68) (width 0.25) (layer "F.Cu") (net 6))
 (segment (start 132.566701 105.315) (end 130.715 105.315) (width 0.25) (layer "F.Cu") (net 6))
 (segment (start 133.931701 106.68) (end 132.566701 105.315) (width 0.25) (layer "F.Cu") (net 6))
 (segment (start 130.715 105.315) (end 129.54 104.14) (width 0.25) (layer "F.Cu") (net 6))
 (segment (start 129.54 93.98) (end 193.04 93.98) (width 0.25) (layer "F.Cu") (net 6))
 (segment (start 193.04 93.98) (end 200.66 101.6) (width 0.25) (layer "F.Cu") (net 6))
 (via (at 200.66 121.92) (size 0.8) (drill 0.4) (layers "F.Cu" "B.Cu") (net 6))
 (via (at 200.66 101.6) (size 0.8) (drill 0.4) (layers "F.Cu" "B.Cu") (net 6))
 (segment (start 200.66 101.6) (end 200.66 121.92) (width 0.25) (layer "B.Cu") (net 6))
 (segment (start 135.106701 105.505) (end 133.445 105.505) (width 0.25) (layer "F.Cu") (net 11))
 (segment (start 133.445 105.505) (end 132.08 104.14) (width 0.25) (layer "F.Cu") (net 11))
 (segment (start 160.02 130.418299) (end 135.106701 105.505) (width 0.25) (layer "F.Cu") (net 11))
 (segment (start 192.8775 137.16) (end 160.02 137.16) (width 0.25) (layer "F.Cu") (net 11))
 (segment (start 192.0775 136.36) (end 192.8775 137.16) (width 0.25) (layer "F.Cu") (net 11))
 (segment (start 160.02 137.16) (end 160.02 130.418299) (width 0.25) (layer "F.Cu") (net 11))
 (segment (start 135.106701 108.045) (end 133.445 108.045) (width 0.25) (layer "F.Cu") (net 12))
 (segment (start 192.0775 138.9) (end 159.22 138.9) (width 0.25) (layer "F.Cu") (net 12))
 (segment (start 159.22 138.9) (end 157.48 137.16) (width 0.25) (layer "F.Cu") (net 12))
 (segment (start 133.445 108.045) (end 132.08 106.68) (width 0.25) (layer "F.Cu") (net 12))
 (segment (start 157.48 130.418299) (end 135.106701 108.045) (width 0.25) (layer "F.Cu") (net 12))
 (segment (start 157.48 137.16) (end 157.48 130.418299) (width 0.25) (layer "F.Cu") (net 12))
 (segment (start 150.31 137.61) (end 150.31 127.45) (width 0.25) (layer "F.Cu") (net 13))
 (segment (start 154.94 142.24) (end 150.31 137.61) (width 0.25) (layer "F.Cu") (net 13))
 (segment (start 150.31 127.45) (end 138.525 115.665) (width 0.25) (layer "F.Cu") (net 13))
 (segment (start 192.0775 141.44) (end 192.8775 142.24) (width 0.25) (layer "F.Cu") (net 13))
 (segment (start 133.255 115.664999) (end 133.255 110.585) (width 0.25) (layer "F.Cu") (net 13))
 (segment (start 192.8775 142.24) (end 154.94 142.24) (width 0.25) (layer "F.Cu") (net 13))
 (segment (start 138.525 115.665) (end 133.255 115.664999) (width 0.25) (layer "F.Cu") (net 13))
 (segment (start 133.255 110.585) (end 134.62 109.22) (width 0.25) (layer "F.Cu") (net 13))
 (segment (start 149.86 127.878299) (end 140.186701 118.205) (width 0.25) (layer "F.Cu") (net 14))
 (segment (start 149.86 139.7) (end 149.86 127.878299) (width 0.25) (layer "F.Cu") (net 14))
 (segment (start 131.783299 118.205) (end 129.54 115.961701) (width 0.25) (layer "F.Cu") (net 14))
 (segment (start 154.14 143.98) (end 149.86 139.7) (width 0.25) (layer "F.Cu") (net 14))
 (segment (start 192.0775 143.98) (end 154.14 143.98) (width 0.25) (layer "F.Cu") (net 14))
 (segment (start 129.54 111.76) (end 132.08 109.22) (width 0.25) (layer "F.Cu") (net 14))
 (segment (start 140.186701 118.205) (end 131.783299 118.205) (width 0.25) (layer "F.Cu") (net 14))
 (segment (start 129.54 115.961701) (end 129.54 111.76) (width 0.25) (layer "F.Cu") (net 14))
 (segment (start 133.255 125.825) (end 134.62 124.46) (width 0.25) (layer "F.Cu") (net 85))
 (segment (start 131.593299 125.825) (end 133.255 125.825) (width 0.25) (layer "F.Cu") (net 85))
 (segment (start 108.19 180.73) (end 108.19 149.228299) (width 0.25) (layer "F.Cu") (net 85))
 (segment (start 108.19 149.228299) (end 131.593299 125.825) (width 0.25) (layer "F.Cu") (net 85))
 (segment (start 72.295 125.635) (end 71.12 124.46) (width 0.25) (layer "F.Cu") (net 41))
 (segment (start 82.645 125.635) (end 72.295 125.635) (width 0.25) (layer "F.Cu") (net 41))
 (segment (start 83.82 124.46) (end 82.645 125.635) (width 0.25) (layer "F.Cu") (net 41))
 (segment (start 45.72 124.46) (end 35.56 124.46) (width 0.25) (layer "F.Cu") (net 62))
 (segment (start 35.56 124.46) (end 33.02 127) (width 0.25) (layer "F.Cu") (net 62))
 (segment (start 180.34 154.94) (end 185.42 149.86) (width 0.25) (layer "F.Cu") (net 3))
 (segment (start 27.94 170.18) (end 33.075 170.18) (width 0.25) (layer "F.Cu") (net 3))
 (segment (start 134.62 154.94) (end 180.34 154.94) (width 0.25) (layer "F.Cu") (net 3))
 (segment (start 192.0775 113.5) (end 186.22 113.5) (width 0.25) (layer "F.Cu") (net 3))
 (segment (start 27.94 170.18) (end 41.965 184.205) (width 0.25) (layer "F.Cu") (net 3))
 (segment (start 186.22 113.5) (end 185.42 114.3) (width 0.25) (layer "F.Cu") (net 3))
 (segment (start 118.415 184.205) (end 133.445 169.175) (width 0.25) (layer "F.Cu") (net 3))
 (segment (start 133.445 156.115) (end 134.62 154.94) (width 0.25) (layer "F.Cu") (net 3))
 (segment (start 33.075 170.18) (end 37.305 165.95) (width 0.25) (layer "F.Cu") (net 3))
 (segment (start 133.445 169.175) (end 133.445 156.115) (width 0.25) (layer "F.Cu") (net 3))
 (segment (start 116.84 170.18) (end 132.08 154.94) (width 0.25) (layer "F.Cu") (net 3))
 (segment (start 192.0775 113.5) (end 209.47 113.5) (width 0.25) (layer "F.Cu") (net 3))
 (segment (start 116.84 178.58) (end 116.84 170.18) (width 0.25) (layer "F.Cu") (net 3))
 (segment (start 41.965 184.205) (end 118.415 184.205) (width 0.25) (layer "F.Cu") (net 3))
 (segment (start 209.47 113.5) (end 215.535 107.435) (width 0.25) (layer "F.Cu") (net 3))
 (via (at 185.42 114.3) (size 0.8) (drill 0.4) (layers "F.Cu" "B.Cu") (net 3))
 (via (at 185.42 149.86) (size 0.8) (drill 0.4) (layers "F.Cu" "B.Cu") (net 3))
 (segment (start 185.42 114.3) (end 185.42 149.86) (width 0.25) (layer "B.Cu") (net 3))
 (segment (start 192.0775 108.42) (end 186.22 108.42) (width 0.25) (layer "F.Cu") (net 2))
 (segment (start 133.445 151.035) (end 138.525 151.035) (width 0.25) (layer "F.Cu") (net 2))
 (segment (start 132.08 152.4) (end 133.445 151.035) (width 0.25) (layer "F.Cu") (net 2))
 (segment (start 138.525 151.035) (end 147.32 142.24) (width 0.25) (layer "F.Cu") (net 2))
 (segment (start 186.22 108.42) (end 177.8 116.84) (width 0.25) (layer "F.Cu") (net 2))
 (via (at 147.32 142.24) (size 0.8) (drill 0.4) (layers "F.Cu" "B.Cu") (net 2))
 (via (at 177.8 116.84) (size 0.8) (drill 0.4) (layers "F.Cu" "B.Cu") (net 2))
 (segment (start 147.32 142.24) (end 172.72 116.84) (width 0.25) (layer "B.Cu") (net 2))
 (segment (start 172.72 116.84) (end 177.8 116.84) (width 0.25) (layer "B.Cu") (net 2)))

